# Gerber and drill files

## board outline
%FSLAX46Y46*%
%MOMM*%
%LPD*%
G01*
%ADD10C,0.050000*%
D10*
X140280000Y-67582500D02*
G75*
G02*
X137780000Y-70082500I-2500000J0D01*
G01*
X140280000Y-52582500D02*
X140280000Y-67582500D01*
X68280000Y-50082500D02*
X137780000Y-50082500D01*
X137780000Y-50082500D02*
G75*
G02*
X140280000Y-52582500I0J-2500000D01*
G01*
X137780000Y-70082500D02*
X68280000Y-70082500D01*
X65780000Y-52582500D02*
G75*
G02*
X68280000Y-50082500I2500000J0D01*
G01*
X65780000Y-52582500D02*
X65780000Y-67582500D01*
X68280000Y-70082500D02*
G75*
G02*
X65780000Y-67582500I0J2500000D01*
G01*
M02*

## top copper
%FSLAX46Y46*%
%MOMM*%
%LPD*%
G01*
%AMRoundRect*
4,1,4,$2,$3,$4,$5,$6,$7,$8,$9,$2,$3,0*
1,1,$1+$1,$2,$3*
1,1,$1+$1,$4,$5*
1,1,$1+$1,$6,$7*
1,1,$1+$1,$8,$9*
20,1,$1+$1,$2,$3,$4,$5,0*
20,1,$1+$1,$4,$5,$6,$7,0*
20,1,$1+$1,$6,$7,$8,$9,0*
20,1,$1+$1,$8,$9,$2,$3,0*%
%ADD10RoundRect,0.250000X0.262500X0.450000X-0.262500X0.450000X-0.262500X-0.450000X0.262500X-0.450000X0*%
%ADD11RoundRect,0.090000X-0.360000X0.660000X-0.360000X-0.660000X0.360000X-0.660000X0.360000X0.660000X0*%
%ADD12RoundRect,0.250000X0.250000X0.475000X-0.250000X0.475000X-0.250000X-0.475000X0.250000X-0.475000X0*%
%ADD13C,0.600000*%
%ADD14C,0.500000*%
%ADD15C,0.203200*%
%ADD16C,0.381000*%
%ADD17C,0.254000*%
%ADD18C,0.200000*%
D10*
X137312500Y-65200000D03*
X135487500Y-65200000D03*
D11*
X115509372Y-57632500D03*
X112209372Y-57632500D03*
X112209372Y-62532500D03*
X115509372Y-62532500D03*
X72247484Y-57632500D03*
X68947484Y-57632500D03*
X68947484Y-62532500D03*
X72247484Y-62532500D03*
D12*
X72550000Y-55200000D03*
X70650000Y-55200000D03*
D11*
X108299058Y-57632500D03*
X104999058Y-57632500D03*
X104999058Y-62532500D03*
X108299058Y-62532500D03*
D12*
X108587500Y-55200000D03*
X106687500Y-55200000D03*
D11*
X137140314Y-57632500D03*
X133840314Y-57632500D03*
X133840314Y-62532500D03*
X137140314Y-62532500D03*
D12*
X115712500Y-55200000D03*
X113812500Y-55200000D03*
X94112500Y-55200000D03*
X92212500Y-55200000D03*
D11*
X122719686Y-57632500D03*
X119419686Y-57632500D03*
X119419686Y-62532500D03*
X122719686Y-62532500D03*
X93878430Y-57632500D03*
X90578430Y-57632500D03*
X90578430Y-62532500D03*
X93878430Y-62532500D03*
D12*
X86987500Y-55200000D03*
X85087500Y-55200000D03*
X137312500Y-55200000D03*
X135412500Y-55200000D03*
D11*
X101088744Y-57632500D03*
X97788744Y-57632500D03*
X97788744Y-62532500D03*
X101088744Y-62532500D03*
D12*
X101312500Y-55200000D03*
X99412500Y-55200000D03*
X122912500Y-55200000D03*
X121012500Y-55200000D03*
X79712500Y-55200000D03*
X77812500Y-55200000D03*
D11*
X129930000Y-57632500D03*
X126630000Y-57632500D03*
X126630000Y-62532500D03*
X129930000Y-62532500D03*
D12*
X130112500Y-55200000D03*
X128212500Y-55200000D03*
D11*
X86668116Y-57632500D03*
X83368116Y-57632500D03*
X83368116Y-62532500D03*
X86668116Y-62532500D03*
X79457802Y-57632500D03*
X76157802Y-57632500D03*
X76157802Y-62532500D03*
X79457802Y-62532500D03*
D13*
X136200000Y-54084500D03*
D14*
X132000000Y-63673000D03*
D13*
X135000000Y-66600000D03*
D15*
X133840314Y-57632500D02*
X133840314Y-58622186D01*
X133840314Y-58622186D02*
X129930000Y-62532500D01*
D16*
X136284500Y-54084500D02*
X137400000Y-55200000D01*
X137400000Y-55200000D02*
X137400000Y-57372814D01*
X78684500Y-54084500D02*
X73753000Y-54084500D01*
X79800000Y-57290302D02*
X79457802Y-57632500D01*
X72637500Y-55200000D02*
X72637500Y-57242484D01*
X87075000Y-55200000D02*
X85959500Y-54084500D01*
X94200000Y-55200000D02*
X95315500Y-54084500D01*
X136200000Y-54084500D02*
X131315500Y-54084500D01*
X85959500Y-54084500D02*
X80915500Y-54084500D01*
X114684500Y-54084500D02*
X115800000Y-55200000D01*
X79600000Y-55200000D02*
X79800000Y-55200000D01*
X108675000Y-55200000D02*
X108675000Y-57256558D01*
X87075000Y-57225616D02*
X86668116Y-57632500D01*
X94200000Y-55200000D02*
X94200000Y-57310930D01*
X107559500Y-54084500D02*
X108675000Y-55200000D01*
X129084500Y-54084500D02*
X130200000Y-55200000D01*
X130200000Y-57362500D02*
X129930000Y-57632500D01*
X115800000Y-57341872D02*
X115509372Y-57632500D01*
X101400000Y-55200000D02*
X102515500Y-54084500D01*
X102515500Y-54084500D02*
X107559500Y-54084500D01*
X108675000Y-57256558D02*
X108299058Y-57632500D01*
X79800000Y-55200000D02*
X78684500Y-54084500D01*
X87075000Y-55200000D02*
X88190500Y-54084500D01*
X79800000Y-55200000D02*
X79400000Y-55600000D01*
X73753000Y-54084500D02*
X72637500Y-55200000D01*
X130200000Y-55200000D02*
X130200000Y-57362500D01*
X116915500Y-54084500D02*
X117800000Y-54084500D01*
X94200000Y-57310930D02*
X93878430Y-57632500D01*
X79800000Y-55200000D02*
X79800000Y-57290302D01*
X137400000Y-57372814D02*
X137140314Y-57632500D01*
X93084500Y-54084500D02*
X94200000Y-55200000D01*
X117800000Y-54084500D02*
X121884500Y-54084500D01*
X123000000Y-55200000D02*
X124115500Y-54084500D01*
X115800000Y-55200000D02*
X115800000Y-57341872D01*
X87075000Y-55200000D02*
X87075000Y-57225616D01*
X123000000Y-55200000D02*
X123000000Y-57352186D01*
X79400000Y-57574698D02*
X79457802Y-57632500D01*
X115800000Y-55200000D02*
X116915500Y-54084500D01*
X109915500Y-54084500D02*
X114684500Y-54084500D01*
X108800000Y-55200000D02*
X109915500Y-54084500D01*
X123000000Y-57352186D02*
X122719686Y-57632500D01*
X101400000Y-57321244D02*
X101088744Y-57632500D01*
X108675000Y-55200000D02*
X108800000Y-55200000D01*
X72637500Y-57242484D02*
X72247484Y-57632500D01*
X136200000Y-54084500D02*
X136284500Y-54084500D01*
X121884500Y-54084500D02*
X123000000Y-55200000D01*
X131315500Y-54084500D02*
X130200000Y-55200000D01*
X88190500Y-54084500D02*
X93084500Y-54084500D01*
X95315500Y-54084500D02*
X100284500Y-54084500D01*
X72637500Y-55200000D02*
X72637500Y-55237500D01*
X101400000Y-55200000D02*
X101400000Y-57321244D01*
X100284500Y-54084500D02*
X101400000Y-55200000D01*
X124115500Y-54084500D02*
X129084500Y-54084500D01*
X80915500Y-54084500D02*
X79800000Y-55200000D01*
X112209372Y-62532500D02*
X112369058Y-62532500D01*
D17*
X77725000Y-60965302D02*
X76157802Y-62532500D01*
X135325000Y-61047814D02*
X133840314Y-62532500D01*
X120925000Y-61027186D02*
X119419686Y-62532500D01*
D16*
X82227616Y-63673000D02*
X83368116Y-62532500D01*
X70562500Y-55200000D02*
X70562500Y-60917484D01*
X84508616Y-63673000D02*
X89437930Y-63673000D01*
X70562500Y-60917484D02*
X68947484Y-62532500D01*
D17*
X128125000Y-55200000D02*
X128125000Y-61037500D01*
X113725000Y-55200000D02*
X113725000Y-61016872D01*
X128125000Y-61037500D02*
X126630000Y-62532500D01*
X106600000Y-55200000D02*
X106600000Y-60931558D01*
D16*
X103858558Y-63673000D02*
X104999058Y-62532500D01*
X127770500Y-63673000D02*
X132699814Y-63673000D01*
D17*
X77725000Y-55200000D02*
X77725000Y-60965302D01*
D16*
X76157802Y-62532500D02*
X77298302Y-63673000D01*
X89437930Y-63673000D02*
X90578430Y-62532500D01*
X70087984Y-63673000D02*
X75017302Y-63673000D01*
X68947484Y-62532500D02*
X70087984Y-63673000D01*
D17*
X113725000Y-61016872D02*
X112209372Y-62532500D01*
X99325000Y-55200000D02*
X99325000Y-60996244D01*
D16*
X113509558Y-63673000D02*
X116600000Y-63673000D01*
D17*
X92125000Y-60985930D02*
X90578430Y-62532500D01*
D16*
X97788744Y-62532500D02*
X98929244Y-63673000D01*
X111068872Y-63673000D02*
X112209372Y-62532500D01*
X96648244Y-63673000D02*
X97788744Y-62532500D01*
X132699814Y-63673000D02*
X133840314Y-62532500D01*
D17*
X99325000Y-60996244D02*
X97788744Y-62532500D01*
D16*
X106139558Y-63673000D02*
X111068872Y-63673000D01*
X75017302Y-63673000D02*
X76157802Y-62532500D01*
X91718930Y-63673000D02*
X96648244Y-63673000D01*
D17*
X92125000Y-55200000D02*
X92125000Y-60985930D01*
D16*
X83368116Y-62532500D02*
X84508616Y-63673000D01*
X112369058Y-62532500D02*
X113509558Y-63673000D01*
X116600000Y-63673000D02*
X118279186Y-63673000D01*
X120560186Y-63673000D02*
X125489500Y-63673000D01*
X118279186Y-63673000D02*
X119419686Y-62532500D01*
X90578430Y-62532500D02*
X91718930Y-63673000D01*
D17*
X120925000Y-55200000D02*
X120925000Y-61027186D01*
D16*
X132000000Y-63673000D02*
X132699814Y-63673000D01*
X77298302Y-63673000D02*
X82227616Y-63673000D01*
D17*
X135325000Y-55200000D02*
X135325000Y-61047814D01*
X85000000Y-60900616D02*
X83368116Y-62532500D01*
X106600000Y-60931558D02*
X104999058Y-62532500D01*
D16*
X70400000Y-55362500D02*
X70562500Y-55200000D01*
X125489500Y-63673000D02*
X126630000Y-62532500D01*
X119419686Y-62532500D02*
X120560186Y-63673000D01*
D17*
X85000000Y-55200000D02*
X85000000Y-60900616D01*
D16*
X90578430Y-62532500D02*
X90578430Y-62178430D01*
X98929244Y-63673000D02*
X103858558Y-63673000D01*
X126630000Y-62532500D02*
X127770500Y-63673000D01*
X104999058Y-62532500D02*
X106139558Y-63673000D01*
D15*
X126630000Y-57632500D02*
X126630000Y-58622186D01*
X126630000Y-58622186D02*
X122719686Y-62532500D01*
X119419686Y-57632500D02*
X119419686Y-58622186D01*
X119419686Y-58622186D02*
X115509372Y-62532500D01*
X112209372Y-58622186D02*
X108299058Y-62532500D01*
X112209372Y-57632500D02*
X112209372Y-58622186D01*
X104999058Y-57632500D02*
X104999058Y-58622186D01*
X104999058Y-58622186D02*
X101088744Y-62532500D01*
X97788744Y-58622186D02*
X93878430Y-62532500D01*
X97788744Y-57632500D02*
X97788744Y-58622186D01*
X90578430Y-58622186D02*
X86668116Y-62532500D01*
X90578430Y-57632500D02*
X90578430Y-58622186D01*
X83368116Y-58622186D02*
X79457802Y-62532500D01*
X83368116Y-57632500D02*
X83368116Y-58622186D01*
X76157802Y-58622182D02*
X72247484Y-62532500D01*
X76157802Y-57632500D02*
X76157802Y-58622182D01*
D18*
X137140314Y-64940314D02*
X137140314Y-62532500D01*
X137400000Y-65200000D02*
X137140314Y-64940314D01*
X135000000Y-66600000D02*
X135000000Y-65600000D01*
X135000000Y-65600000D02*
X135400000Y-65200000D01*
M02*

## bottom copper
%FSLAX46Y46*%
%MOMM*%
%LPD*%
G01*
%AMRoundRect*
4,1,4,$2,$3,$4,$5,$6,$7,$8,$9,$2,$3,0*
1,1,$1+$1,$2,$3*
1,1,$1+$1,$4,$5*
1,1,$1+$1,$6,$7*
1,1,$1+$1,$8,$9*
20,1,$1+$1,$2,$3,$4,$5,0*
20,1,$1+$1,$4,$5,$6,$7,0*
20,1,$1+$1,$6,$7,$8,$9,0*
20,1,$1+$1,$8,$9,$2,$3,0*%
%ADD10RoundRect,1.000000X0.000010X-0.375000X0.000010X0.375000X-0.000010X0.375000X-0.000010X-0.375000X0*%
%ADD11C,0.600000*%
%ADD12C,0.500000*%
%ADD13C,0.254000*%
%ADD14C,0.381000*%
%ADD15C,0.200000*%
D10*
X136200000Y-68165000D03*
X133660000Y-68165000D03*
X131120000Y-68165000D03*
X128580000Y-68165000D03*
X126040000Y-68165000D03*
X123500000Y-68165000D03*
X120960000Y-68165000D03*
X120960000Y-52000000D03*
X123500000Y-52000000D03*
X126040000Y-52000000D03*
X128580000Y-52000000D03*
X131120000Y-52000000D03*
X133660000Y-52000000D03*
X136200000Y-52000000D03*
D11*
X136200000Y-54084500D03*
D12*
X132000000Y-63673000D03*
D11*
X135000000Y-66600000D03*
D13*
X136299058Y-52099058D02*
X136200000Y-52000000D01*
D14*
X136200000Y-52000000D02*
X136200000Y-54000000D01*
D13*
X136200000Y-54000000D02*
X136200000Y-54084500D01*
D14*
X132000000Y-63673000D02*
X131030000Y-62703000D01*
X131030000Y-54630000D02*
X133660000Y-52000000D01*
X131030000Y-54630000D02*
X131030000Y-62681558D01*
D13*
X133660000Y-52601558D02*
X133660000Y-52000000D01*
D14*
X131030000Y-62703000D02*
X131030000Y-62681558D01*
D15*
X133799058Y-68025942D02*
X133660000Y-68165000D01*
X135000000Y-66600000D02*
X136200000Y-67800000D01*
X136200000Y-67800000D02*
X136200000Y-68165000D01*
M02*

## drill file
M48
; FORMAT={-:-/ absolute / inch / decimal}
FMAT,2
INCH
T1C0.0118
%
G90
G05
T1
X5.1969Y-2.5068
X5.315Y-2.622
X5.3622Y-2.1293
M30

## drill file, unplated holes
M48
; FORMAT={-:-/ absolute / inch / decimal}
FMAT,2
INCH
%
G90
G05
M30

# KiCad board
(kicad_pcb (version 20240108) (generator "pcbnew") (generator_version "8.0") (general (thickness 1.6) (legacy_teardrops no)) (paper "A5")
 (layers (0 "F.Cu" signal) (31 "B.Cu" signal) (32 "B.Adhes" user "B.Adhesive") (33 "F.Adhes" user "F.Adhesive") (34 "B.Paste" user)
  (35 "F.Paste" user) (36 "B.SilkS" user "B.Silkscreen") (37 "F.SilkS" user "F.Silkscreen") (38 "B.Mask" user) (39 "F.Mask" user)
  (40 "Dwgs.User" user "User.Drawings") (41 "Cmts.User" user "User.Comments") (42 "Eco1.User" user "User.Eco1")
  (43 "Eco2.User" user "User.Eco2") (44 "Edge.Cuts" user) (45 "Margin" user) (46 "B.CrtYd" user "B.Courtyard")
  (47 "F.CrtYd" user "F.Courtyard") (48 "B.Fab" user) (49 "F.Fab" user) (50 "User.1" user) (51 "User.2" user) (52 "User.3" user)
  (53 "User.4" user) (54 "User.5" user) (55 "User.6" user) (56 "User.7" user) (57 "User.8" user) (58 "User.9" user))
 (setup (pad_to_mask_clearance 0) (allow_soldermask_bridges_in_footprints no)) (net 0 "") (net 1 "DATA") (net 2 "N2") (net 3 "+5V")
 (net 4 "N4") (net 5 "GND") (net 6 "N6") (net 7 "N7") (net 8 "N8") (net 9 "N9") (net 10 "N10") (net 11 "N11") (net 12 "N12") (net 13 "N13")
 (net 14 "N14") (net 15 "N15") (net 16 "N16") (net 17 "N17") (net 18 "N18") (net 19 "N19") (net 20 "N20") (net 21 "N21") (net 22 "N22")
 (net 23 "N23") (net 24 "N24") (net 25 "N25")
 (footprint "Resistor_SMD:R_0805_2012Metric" (layer "F.Cu") (at 136.4 65.2 180)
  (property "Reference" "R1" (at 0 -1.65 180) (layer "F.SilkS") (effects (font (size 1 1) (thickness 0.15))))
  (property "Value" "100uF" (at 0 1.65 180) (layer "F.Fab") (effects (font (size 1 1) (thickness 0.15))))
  (pad "1" smd roundrect (at -0.9125 0 180) (size 1.025 1.4) (layers "F.Cu" "F.Paste" "F.Mask") (roundrect_rratio 0.243902) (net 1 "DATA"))
  (pad "2" smd roundrect (at 0.9125 0 180) (size 1.025 1.4) (layers "F.Cu" "F.Paste" "F.Mask") (roundrect_rratio 0.243902) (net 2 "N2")))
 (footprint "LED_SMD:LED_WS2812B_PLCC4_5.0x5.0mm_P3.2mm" (layer "F.Cu") (at 113.859372 60.0825 -90)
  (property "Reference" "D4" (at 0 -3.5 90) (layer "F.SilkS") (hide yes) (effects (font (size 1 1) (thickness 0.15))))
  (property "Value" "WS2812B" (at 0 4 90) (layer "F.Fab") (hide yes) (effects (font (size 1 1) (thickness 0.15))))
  (pad "1" smd roundrect (at -2.45 -1.65 270) (size 1.5 0.9) (layers "F.Cu" "F.Paste" "F.Mask") (roundrect_rratio 0.1) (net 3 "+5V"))
  (pad "2" smd roundrect (at -2.45 1.65 270) (size 1.5 0.9) (layers "F.Cu" "F.Paste" "F.Mask") (roundrect_rratio 0.1) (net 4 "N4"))
  (pad "3" smd roundrect (at 2.45 1.65 270) (size 1.5 0.9) (layers "F.Cu" "F.Paste" "F.Mask") (roundrect_rratio 0.1) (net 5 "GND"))
  (pad "4" smd roundrect (at 2.45 -1.65 270) (size 1.5 0.9) (layers "F.Cu" "F.Paste" "F.Mask") (roundrect_rratio 0.1) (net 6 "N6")))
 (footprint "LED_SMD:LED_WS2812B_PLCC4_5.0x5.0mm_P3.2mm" (layer "F.Cu") (at 70.597484 60.0825 -90)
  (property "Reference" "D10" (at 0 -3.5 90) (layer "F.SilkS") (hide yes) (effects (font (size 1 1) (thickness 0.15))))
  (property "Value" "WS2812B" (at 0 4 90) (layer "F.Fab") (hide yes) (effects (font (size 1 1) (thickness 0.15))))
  (pad "1" smd roundrect (at -2.45 -1.65 270) (size 1.5 0.9) (layers "F.Cu" "F.Paste" "F.Mask") (roundrect_rratio 0.1) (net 3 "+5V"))
  (pad "2" smd roundrect (at -2.45 1.65 270) (size 1.5 0.9) (layers "F.Cu" "F.Paste" "F.Mask") (roundrect_rratio 0.1) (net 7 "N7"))
  (pad "3" smd roundrect (at 2.45 1.65 270) (size 1.5 0.9) (layers "F.Cu" "F.Paste" "F.Mask") (roundrect_rratio 0.1) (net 5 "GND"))
  (pad "4" smd roundrect (at 2.45 -1.65 270) (size 1.5 0.9) (layers "F.Cu" "F.Paste" "F.Mask") (roundrect_rratio 0.1) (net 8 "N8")))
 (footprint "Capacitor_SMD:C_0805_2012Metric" (layer "F.Cu") (at 71.6 55.2 180)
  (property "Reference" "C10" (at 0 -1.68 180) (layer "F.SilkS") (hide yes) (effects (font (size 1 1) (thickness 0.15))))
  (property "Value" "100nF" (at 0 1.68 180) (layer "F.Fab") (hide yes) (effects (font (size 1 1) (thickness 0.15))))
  (pad "1" smd roundrect (at -0.95 0 180) (size 1 1.45) (layers "F.Cu" "F.Paste" "F.Mask") (roundrect_rratio 0.25) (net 3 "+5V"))
  (pad "2" smd roundrect (at 0.95 0 180) (size 1 1.45) (layers "F.Cu" "F.Paste" "F.Mask") (roundrect_rratio 0.25) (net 5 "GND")))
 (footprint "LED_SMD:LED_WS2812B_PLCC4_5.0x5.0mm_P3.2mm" (layer "F.Cu") (at 106.649058 60.0825 -90)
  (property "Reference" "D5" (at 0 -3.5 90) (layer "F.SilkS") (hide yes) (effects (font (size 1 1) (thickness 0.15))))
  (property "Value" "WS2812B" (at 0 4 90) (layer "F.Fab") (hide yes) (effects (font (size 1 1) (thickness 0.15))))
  (pad "1" smd roundrect (at -2.45 -1.65 270) (size 1.5 0.9) (layers "F.Cu" "F.Paste" "F.Mask") (roundrect_rratio 0.1) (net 3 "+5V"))
  (pad "2" smd roundrect (at -2.45 1.65 270) (size 1.5 0.9) (layers "F.Cu" "F.Paste" "F.Mask") (roundrect_rratio 0.1) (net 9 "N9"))
  (pad "3" smd roundrect (at 2.45 1.65 270) (size 1.5 0.9) (layers "F.Cu" "F.Paste" "F.Mask") (roundrect_rratio 0.1) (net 5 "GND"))
  (pad "4" smd roundrect (at 2.45 -1.65 270) (size 1.5 0.9) (layers "F.Cu" "F.Paste" "F.Mask") (roundrect_rratio 0.1) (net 4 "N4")))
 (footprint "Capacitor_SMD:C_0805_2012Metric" (layer "F.Cu") (at 107.6375 55.2 180)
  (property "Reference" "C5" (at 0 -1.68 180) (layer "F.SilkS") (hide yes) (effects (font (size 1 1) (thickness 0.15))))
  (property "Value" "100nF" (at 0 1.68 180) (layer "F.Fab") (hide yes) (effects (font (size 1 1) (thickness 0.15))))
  (pad "1" smd roundrect (at -0.95 0 180) (size 1 1.45) (layers "F.Cu" "F.Paste" "F.Mask") (roundrect_rratio 0.25) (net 3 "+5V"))
  (pad "2" smd roundrect (at 0.95 0 180) (size 1 1.45) (layers "F.Cu" "F.Paste" "F.Mask") (roundrect_rratio 0.25) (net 5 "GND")))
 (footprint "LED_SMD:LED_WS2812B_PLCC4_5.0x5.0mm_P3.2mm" (layer "F.Cu") (at 135.490314 60.0825 -90)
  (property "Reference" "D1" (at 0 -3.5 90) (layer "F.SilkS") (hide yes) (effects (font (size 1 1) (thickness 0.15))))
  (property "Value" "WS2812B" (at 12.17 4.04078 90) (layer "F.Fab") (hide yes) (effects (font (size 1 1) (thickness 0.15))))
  (pad "1" smd roundrect (at -2.45 -1.65 270) (size 1.5 0.9) (layers "F.Cu" "F.Paste" "F.Mask") (roundrect_rratio 0.1) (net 3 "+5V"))
  (pad "2" smd roundrect (at -2.45 1.65 270) (size 1.5 0.9) (layers "F.Cu" "F.Paste" "F.Mask") (roundrect_rratio 0.1) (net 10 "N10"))
  (pad "3" smd roundrect (at 2.45 1.65 270) (size 1.5 0.9) (layers "F.Cu" "F.Paste" "F.Mask") (roundrect_rratio 0.1) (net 5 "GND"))
  (pad "4" smd roundrect (at 2.45 -1.65 270) (size 1.5 0.9) (layers "F.Cu" "F.Paste" "F.Mask") (roundrect_rratio 0.1) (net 1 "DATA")))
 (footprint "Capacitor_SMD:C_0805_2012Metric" (layer "F.Cu") (at 114.7625 55.2 180)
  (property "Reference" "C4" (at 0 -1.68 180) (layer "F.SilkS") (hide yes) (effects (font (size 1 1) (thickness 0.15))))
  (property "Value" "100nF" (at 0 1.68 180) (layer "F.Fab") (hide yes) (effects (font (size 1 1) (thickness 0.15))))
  (pad "1" smd roundrect (at -0.95 0 180) (size 1 1.45) (layers "F.Cu" "F.Paste" "F.Mask") (roundrect_rratio 0.25) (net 3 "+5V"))
  (pad "2" smd roundrect (at 0.95 0 180) (size 1 1.45) (layers "F.Cu" "F.Paste" "F.Mask") (roundrect_rratio 0.25) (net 5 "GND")))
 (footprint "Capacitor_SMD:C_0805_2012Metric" (layer "F.Cu") (at 93.1625 55.2 180)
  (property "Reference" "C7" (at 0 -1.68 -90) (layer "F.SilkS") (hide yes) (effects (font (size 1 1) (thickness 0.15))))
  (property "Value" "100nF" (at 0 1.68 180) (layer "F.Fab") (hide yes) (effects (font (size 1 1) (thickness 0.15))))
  (pad "1" smd roundrect (at -0.95 0 180) (size 1 1.45) (layers "F.Cu" "F.Paste" "F.Mask") (roundrect_rratio 0.25) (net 3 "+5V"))
  (pad "2" smd roundrect (at 0.95 0 180) (size 1 1.45) (layers "F.Cu" "F.Paste" "F.Mask") (roundrect_rratio 0.25) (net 5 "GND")))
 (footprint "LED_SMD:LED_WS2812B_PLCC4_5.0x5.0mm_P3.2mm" (layer "F.Cu") (at 121.069686 60.0825 -90)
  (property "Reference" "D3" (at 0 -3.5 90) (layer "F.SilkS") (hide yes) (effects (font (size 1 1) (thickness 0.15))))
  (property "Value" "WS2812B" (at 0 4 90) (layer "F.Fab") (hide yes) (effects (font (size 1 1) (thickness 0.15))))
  (pad "1" smd roundrect (at -2.45 -1.65 270) (size 1.5 0.9) (layers "F.Cu" "F.Paste" "F.Mask") (roundrect_rratio 0.1) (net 3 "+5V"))
  (pad "2" smd roundrect (at -2.45 1.65 270) (size 1.5 0.9) (layers "F.Cu" "F.Paste" "F.Mask") (roundrect_rratio 0.1) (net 6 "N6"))
  (pad "3" smd roundrect (at 2.45 1.65 270) (size 1.5 0.9) (layers "F.Cu" "F.Paste" "F.Mask") (roundrect_rratio 0.1) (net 5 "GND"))
  (pad "4" smd roundrect (at 2.45 -1.65 270) (size 1.5 0.9) (layers "F.Cu" "F.Paste" "F.Mask") (roundrect_rratio 0.1) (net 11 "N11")))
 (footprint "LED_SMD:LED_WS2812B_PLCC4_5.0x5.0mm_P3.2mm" (layer "F.Cu") (at 92.22843 60.0825 -90)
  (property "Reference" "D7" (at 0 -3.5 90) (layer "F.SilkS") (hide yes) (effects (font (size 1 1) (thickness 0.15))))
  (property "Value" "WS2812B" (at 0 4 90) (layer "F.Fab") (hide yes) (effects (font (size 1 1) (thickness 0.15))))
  (pad "1" smd roundrect (at -2.45 -1.65 270) (size 1.5 0.9) (layers "F.Cu" "F.Paste" "F.Mask") (roundrect_rratio 0.1) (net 3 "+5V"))
  (pad "2" smd roundrect (at -2.45 1.65 270) (size 1.5 0.9) (layers "F.Cu" "F.Paste" "F.Mask") (roundrect_rratio 0.1) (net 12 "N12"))
  (pad "3" smd roundrect (at 2.45 1.65 270) (size 1.5 0.9) (layers "F.Cu" "F.Paste" "F.Mask") (roundrect_rratio 0.1) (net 5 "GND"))
  (pad "4" smd roundrect (at 2.45 -1.65 270) (size 1.5 0.9) (layers "F.Cu" "F.Paste" "F.Mask") (roundrect_rratio 0.1) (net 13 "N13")))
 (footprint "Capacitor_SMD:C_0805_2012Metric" (layer "F.Cu") (at 86.0375 55.2 180)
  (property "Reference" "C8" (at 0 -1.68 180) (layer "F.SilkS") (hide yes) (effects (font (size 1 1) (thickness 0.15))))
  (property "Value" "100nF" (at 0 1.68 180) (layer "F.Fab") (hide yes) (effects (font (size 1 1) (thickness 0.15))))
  (pad "1" smd roundrect (at -0.95 0 180) (size 1 1.45) (layers "F.Cu" "F.Paste" "F.Mask") (roundrect_rratio 0.25) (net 3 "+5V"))
  (pad "2" smd roundrect (at 0.95 0 180) (size 1 1.45) (layers "F.Cu" "F.Paste" "F.Mask") (roundrect_rratio 0.25) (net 5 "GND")))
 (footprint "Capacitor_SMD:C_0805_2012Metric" (layer "F.Cu") (at 136.3625 55.2 180)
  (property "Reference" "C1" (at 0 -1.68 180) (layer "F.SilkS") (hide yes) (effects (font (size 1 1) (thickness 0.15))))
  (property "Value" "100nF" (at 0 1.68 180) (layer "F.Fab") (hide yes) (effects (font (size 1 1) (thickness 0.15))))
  (pad "1" smd roundrect (at -0.95 0 180) (size 1 1.45) (layers "F.Cu" "F.Paste" "F.Mask") (roundrect_rratio 0.25) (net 3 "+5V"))
  (pad "2" smd roundrect (at 0.95 0 180) (size 1 1.45) (layers "F.Cu" "F.Paste" "F.Mask") (roundrect_rratio 0.25) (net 5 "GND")))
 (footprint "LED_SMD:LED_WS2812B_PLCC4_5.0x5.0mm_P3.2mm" (layer "F.Cu") (at 99.438744 60.0825 -90)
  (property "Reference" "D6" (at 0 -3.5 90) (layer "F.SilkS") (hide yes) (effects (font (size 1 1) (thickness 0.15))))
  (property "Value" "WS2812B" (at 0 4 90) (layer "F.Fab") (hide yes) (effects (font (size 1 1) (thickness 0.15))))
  (pad "1" smd roundrect (at -2.45 -1.65 270) (size 1.5 0.9) (layers "F.Cu" "F.Paste" "F.Mask") (roundrect_rratio 0.1) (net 3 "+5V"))
  (pad "2" smd roundrect (at -2.45 1.65 270) (size 1.5 0.9) (layers "F.Cu" "F.Paste" "F.Mask") (roundrect_rratio 0.1) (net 13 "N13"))
  (pad "3" smd roundrect (at 2.45 1.65 270) (size 1.5 0.9) (layers "F.Cu" "F.Paste" "F.Mask") (roundrect_rratio 0.1) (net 5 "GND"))
  (pad "4" smd roundrect (at 2.45 -1.65 270) (size 1.5 0.9) (layers "F.Cu" "F.Paste" "F.Mask") (roundrect_rratio 0.1) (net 9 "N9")))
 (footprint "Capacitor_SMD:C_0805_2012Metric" (layer "F.Cu") (at 100.3625 55.2 180)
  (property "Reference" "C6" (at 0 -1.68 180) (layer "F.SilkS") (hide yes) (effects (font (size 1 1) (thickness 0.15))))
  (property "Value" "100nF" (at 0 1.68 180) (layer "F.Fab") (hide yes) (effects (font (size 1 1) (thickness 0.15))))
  (pad "1" smd roundrect (at -0.95 0 180) (size 1 1.45) (layers "F.Cu" "F.Paste" "F.Mask") (roundrect_rratio 0.25) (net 3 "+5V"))
  (pad "2" smd roundrect (at 0.95 0 180) (size 1 1.45) (layers "F.Cu" "F.Paste" "F.Mask") (roundrect_rratio 0.25) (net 5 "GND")))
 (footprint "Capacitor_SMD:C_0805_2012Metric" (layer "F.Cu") (at 121.9625 55.2 180)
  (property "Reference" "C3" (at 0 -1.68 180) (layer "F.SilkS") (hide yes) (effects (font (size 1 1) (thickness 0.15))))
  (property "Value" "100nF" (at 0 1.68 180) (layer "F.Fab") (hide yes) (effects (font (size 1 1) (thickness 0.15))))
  (pad "1" smd roundrect (at -0.95 0 180) (size 1 1.45) (layers "F.Cu" "F.Paste" "F.Mask") (roundrect_rratio 0.25) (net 3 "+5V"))
  (pad "2" smd roundrect (at 0.95 0 180) (size 1 1.45) (layers "F.Cu" "F.Paste" "F.Mask") (roundrect_rratio 0.25) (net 5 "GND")))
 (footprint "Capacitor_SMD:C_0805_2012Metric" (layer "F.Cu") (at 78.7625 55.2 180)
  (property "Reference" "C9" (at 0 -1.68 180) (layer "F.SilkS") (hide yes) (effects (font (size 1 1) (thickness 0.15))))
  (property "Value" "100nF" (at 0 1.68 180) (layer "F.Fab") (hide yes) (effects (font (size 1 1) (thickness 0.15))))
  (pad "1" smd roundrect (at -0.95 0 180) (size 1 1.45) (layers "F.Cu" "F.Paste" "F.Mask") (roundrect_rratio 0.25) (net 3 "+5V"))
  (pad "2" smd roundrect (at 0.95 0 180) (size 1 1.45) (layers "F.Cu" "F.Paste" "F.Mask") (roundrect_rratio 0.25) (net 5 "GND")))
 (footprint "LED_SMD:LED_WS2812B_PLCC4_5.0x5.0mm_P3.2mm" (layer "F.Cu") (at 128.28 60.0825 -90)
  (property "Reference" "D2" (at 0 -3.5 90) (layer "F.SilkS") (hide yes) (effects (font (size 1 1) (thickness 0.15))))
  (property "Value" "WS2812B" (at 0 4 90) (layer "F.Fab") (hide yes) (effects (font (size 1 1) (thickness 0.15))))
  (pad "1" smd roundrect (at -2.45 -1.65 270) (size 1.5 0.9) (layers "F.Cu" "F.Paste" "F.Mask") (roundrect_rratio 0.1) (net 3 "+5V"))
  (pad "2" smd roundrect (at -2.45 1.65 270) (size 1.5 0.9) (layers "F.Cu" "F.Paste" "F.Mask") (roundrect_rratio 0.1) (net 11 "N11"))
  (pad "3" smd roundrect (at 2.45 1.65 270) (size 1.5 0.9) (layers "F.Cu" "F.Paste" "F.Mask") (roundrect_rratio 0.1) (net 5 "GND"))
  (pad "4" smd roundrect (at 2.45 -1.65 270) (size 1.5 0.9) (layers "F.Cu" "F.Paste" "F.Mask") (roundrect_rratio 0.1) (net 10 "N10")))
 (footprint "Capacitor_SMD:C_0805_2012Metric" (layer "F.Cu") (at 129.1625 55.2 180)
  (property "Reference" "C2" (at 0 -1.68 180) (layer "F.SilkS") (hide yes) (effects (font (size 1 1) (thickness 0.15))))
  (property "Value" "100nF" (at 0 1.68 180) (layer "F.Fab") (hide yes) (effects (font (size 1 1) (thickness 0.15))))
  (pad "1" smd roundrect (at -0.95 0 180) (size 1 1.45) (layers "F.Cu" "F.Paste" "F.Mask") (roundrect_rratio 0.25) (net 3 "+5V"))
  (pad "2" smd roundrect (at 0.95 0 180) (size 1 1.45) (layers "F.Cu" "F.Paste" "F.Mask") (roundrect_rratio 0.25) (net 5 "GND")))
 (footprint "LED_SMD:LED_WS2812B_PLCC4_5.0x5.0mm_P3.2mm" (layer "F.Cu") (at 85.018116 60.0825 -90)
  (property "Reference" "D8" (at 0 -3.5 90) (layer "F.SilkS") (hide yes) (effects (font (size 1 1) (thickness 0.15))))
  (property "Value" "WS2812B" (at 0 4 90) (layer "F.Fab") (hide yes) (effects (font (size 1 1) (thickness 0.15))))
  (pad "1" smd roundrect (at -2.45 -1.65 270) (size 1.5 0.9) (layers "F.Cu" "F.Paste" "F.Mask") (roundrect_rratio 0.1) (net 3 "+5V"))
  (pad "2" smd roundrect (at -2.45 1.65 270) (size 1.5 0.9) (layers "F.Cu" "F.Paste" "F.Mask") (roundrect_rratio 0.1) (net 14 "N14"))
  (pad "3" smd roundrect (at 2.45 1.65 270) (size 1.5 0.9) (layers "F.Cu" "F.Paste" "F.Mask") (roundrect_rratio 0.1) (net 5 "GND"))
  (pad "4" smd roundrect (at 2.45 -1.65 270) (size 1.5 0.9) (layers "F.Cu" "F.Paste" "F.Mask") (roundrect_rratio 0.1) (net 12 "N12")))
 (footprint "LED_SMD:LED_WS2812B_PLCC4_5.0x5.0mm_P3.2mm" (layer "F.Cu") (at 77.807802 60.0825 -90)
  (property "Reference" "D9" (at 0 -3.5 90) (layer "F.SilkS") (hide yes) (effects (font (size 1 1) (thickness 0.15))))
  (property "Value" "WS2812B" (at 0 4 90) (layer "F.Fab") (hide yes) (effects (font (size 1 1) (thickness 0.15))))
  (pad "1" smd roundrect (at -2.45 -1.65 270) (size 1.5 0.9) (layers "F.Cu" "F.Paste" "F.Mask") (roundrect_rratio 0.1) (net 3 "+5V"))
  (pad "2" smd roundrect (at -2.45 1.65 270) (size 1.5 0.9) (layers "F.Cu" "F.Paste" "F.Mask") (roundrect_rratio 0.1) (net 8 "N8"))
  (pad "3" smd roundrect (at 2.45 1.65 270) (size 1.5 0.9) (layers "F.Cu" "F.Paste" "F.Mask") (roundrect_rratio 0.1) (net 5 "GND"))
  (pad "4" smd roundrect (at 2.45 -1.65 270) (size 1.5 0.9) (layers "F.Cu" "F.Paste" "F.Mask") (roundrect_rratio 0.1) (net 14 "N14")))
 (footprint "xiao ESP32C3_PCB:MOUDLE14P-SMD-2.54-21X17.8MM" (layer "B.Cu") (at 118.08 69 90)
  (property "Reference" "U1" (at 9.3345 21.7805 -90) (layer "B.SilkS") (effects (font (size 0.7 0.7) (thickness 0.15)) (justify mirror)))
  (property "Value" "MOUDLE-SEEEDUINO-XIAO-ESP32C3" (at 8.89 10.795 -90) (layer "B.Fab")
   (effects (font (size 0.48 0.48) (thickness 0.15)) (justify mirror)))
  (pad "1" smd roundrect (at 0.835 18.12 90) (size 2.75 2) (layers "B.Cu" "B.Paste" "B.Mask") (roundrect_rratio 0.5) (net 2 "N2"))
  (pad "2" smd roundrect (at 0.835 15.58 90) (size 2.75 2) (layers "B.Cu" "B.Paste" "B.Mask") (roundrect_rratio 0.5) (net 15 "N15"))
  (pad "3" smd roundrect (at 0.835 13.04 90) (size 2.75 2) (layers "B.Cu" "B.Paste" "B.Mask") (roundrect_rratio 0.5) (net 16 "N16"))
  (pad "4" smd roundrect (at 0.835 10.5 90) (size 2.75 2) (layers "B.Cu" "B.Paste" "B.Mask") (roundrect_rratio 0.5) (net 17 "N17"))
  (pad "5" smd roundrect (at 0.835 7.96 90) (size 2.75 2) (layers "B.Cu" "B.Paste" "B.Mask") (roundrect_rratio 0.5) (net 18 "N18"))
  (pad "6" smd roundrect (at 0.835 5.42 90) (size 2.75 2) (layers "B.Cu" "B.Paste" "B.Mask") (roundrect_rratio 0.5) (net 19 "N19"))
  (pad "7" smd roundrect (at 0.835 2.88 90) (size 2.75 2) (layers "B.Cu" "B.Paste" "B.Mask") (roundrect_rratio 0.5) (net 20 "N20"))
  (pad "8" smd roundrect (at 17 2.88 90) (size 2.75 2) (layers "B.Cu" "B.Paste" "B.Mask") (roundrect_rratio 0.5) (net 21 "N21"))
  (pad "9" smd roundrect (at 17 5.42 90) (size 2.75 2) (layers "B.Cu" "B.Paste" "B.Mask") (roundrect_rratio 0.5) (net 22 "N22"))
  (pad "10" smd roundrect (at 17 7.96 90) (size 2.75 2) (layers "B.Cu" "B.Paste" "B.Mask") (roundrect_rratio 0.5) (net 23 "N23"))
  (pad "11" smd roundrect (at 17 10.5 90) (size 2.75 2) (layers "B.Cu" "B.Paste" "B.Mask") (roundrect_rratio 0.5) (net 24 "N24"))
  (pad "12" smd roundrect (at 17 13.04 90) (size 2.75 2) (layers "B.Cu" "B.Paste" "B.Mask") (roundrect_rratio 0.5) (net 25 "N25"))
  (pad "13" smd roundrect (at 17 15.58 90) (size 2.75 2) (layers "B.Cu" "B.Paste" "B.Mask") (roundrect_rratio 0.5) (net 5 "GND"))
  (pad "14" smd roundrect (at 17 18.12 90) (size 2.75 2) (layers "B.Cu" "B.Paste" "B.Mask") (roundrect_rratio 0.5) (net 3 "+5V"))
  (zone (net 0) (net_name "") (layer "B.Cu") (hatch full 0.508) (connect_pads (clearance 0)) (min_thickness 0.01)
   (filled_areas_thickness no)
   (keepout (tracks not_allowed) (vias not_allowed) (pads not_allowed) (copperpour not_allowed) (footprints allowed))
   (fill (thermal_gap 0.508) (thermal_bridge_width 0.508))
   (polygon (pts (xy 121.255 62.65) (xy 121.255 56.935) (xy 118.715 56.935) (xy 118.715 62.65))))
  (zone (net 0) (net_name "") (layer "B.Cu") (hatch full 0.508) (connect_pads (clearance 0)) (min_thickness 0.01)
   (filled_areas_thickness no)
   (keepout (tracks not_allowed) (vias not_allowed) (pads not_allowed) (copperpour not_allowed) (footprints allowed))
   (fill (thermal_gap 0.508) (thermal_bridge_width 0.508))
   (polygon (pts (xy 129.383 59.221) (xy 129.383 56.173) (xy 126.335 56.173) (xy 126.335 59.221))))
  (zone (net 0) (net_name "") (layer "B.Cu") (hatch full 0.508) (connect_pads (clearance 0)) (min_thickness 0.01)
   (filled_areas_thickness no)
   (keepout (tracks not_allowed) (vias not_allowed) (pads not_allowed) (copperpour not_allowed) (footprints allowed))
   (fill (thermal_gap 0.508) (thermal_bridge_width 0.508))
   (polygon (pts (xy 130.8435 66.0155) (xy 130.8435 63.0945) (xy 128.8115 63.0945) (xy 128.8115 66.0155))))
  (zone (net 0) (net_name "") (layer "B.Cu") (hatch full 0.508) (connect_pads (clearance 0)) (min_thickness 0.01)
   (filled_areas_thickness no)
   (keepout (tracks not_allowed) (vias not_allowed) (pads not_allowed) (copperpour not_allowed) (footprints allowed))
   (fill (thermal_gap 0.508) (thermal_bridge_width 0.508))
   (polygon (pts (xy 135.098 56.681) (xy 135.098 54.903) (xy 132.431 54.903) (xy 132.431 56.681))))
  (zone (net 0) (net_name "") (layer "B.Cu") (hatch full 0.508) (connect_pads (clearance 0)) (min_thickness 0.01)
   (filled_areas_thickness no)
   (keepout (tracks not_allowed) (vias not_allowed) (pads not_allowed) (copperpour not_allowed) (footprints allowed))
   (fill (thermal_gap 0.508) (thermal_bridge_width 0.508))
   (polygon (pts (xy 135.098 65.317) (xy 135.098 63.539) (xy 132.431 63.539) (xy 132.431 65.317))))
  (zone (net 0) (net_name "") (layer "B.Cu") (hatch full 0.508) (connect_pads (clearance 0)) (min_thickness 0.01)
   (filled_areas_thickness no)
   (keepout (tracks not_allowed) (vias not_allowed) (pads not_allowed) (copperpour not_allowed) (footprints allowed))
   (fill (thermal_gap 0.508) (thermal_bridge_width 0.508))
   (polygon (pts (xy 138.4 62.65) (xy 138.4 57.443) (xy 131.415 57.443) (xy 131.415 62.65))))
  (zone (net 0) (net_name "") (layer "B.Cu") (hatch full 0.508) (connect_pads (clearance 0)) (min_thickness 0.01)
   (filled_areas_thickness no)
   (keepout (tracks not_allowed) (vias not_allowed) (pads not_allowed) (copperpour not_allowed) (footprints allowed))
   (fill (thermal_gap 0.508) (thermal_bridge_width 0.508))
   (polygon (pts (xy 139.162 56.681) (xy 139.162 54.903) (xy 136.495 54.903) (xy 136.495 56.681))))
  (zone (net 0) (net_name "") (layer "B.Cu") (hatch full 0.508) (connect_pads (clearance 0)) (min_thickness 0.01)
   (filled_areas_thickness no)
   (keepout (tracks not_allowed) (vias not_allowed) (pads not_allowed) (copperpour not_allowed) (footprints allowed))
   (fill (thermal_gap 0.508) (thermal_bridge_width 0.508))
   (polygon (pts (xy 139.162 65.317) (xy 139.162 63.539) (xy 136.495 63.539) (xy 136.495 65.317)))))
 (gr_arc (start 140.28 67.5825) (mid 139.547767 69.350267) (end 137.78 70.0825) (stroke (width 0.05) (type default)) (layer "Edge.Cuts"))
 (gr_line (start 140.28 52.5825) (end 140.28 67.5825) (stroke (width 0.05) (type default)) (layer "Edge.Cuts"))
 (gr_line (start 68.28 50.0825) (end 137.78 50.0825) (stroke (width 0.05) (type default)) (layer "Edge.Cuts"))
 (gr_arc (start 137.78 50.0825) (mid 139.547767 50.814733) (end 140.28 52.5825) (stroke (width 0.05) (type default)) (layer "Edge.Cuts"))
 (gr_line (start 137.78 70.0825) (end 68.28 70.0825) (stroke (width 0.05) (type default)) (layer "Edge.Cuts"))
 (gr_arc (start 65.78 52.5825) (mid 66.512233 50.814733) (end 68.28 50.0825) (stroke (width 0.05) (type default)) (layer "Edge.Cuts"))
 (gr_line (start 65.78 52.5825) (end 65.78 67.5825) (stroke (width 0.05) (type default)) (layer "Edge.Cuts"))
 (gr_arc (start 68.28 70.0825) (mid 66.512233 69.350267) (end 65.78 67.5825) (stroke (width 0.05) (type default)) (layer "Edge.Cuts"))
 (segment (start 133.840314 57.6325) (end 133.840314 58.622186) (width 0.2032) (layer "F.Cu") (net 10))
 (segment (start 133.840314 58.622186) (end 129.93 62.5325) (width 0.2032) (layer "F.Cu") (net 10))
 (segment (start 136.2845 54.0845) (end 137.4 55.2) (width 0.381) (layer "F.Cu") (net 3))
 (segment (start 137.4 55.2) (end 137.4 57.372814) (width 0.381) (layer "F.Cu") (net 3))
 (segment (start 78.6845 54.0845) (end 73.753 54.0845) (width 0.381) (layer "F.Cu") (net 3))
 (segment (start 79.8 57.290302) (end 79.457802 57.6325) (width 0.381) (layer "F.Cu") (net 3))
 (segment (start 72.6375 55.2) (end 72.6375 57.242484) (width 0.381) (layer "F.Cu") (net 3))
 (segment (start 87.075 55.2) (end 85.9595 54.0845) (width 0.381) (layer "F.Cu") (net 3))
 (segment (start 94.2 55.2) (end 95.3155 54.0845) (width 0.381) (layer "F.Cu") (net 3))
 (segment (start 136.2 54.0845) (end 131.3155 54.0845) (width 0.381) (layer "F.Cu") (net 3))
 (segment (start 85.9595 54.0845) (end 80.9155 54.0845) (width 0.381) (layer "F.Cu") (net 3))
 (segment (start 114.6845 54.0845) (end 115.8 55.2) (width 0.381) (layer "F.Cu") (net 3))
 (segment (start 79.6 55.2) (end 79.8 55.2) (width 0.381) (layer "F.Cu") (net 3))
 (segment (start 108.675 55.2) (end 108.675 57.256558) (width 0.381) (layer "F.Cu") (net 3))
 (segment (start 87.075 57.225616) (end 86.668116 57.6325) (width 0.381) (layer "F.Cu") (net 3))
 (segment (start 94.2 55.2) (end 94.2 57.31093) (width 0.381) (layer "F.Cu") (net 3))
 (segment (start 107.5595 54.0845) (end 108.675 55.2) (width 0.381) (layer "F.Cu") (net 3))
 (segment (start 129.0845 54.0845) (end 130.2 55.2) (width 0.381) (layer "F.Cu") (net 3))
 (segment (start 130.2 57.3625) (end 129.93 57.6325) (width 0.381) (layer "F.Cu") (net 3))
 (segment (start 115.8 57.341872) (end 115.509372 57.6325) (width 0.381) (layer "F.Cu") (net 3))
 (segment (start 101.4 55.2) (end 102.5155 54.0845) (width 0.381) (layer "F.Cu") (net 3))
 (segment (start 102.5155 54.0845) (end 107.5595 54.0845) (width 0.381) (layer "F.Cu") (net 3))
 (segment (start 108.675 57.256558) (end 108.299058 57.6325) (width 0.381) (layer "F.Cu") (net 3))
 (segment (start 79.8 55.2) (end 78.6845 54.0845) (width 0.381) (layer "F.Cu") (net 3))
 (segment (start 87.075 55.2) (end 88.1905 54.0845) (width 0.381) (layer "F.Cu") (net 3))
 (segment (start 79.8 55.2) (end 79.4 55.6) (width 0.381) (layer "F.Cu") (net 3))
 (segment (start 73.753 54.0845) (end 72.6375 55.2) (width 0.381) (layer "F.Cu") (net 3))
 (segment (start 130.2 55.2) (end 130.2 57.3625) (width 0.381) (layer "F.Cu") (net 3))
 (segment (start 116.9155 54.0845) (end 117.8 54.0845) (width 0.381) (layer "F.Cu") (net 3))
 (segment (start 94.2 57.31093) (end 93.87843 57.6325) (width 0.381) (layer "F.Cu") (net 3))
 (segment (start 79.8 55.2) (end 79.8 57.290302) (width 0.381) (layer "F.Cu") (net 3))
 (segment (start 137.4 57.372814) (end 137.140314 57.6325) (width 0.381) (layer "F.Cu") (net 3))
 (segment (start 93.0845 54.0845) (end 94.2 55.2) (width 0.381) (layer "F.Cu") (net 3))
 (segment (start 117.8 54.0845) (end 121.8845 54.0845) (width 0.381) (layer "F.Cu") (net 3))
 (segment (start 123 55.2) (end 124.1155 54.0845) (width 0.381) (layer "F.Cu") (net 3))
 (segment (start 115.8 55.2) (end 115.8 57.341872) (width 0.381) (layer "F.Cu") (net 3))
 (segment (start 87.075 55.2) (end 87.075 57.225616) (width 0.381) (layer "F.Cu") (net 3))
 (segment (start 123 55.2) (end 123 57.352186) (width 0.381) (layer "F.Cu") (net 3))
 (segment (start 79.4 57.574698) (end 79.457802 57.6325) (width 0.381) (layer "F.Cu") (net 3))
 (segment (start 115.8 55.2) (end 116.9155 54.0845) (width 0.381) (layer "F.Cu") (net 3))
 (segment (start 109.9155 54.0845) (end 114.6845 54.0845) (width 0.381) (layer "F.Cu") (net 3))
 (segment (start 108.8 55.2) (end 109.9155 54.0845) (width 0.381) (layer "F.Cu") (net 3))
 (segment (start 123 57.352186) (end 122.719686 57.6325) (width 0.381) (layer "F.Cu") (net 3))
 (segment (start 101.4 57.321244) (end 101.088744 57.6325) (width 0.381) (layer "F.Cu") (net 3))
 (segment (start 108.675 55.2) (end 108.8 55.2) (width 0.381) (layer "F.Cu") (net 3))
 (segment (start 72.6375 57.242484) (end 72.247484 57.6325) (width 0.381) (layer "F.Cu") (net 3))
 (segment (start 136.2 54.0845) (end 136.2845 54.0845) (width 0.381) (layer "F.Cu") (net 3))
 (segment (start 121.8845 54.0845) (end 123 55.2) (width 0.381) (layer "F.Cu") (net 3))
 (segment (start 131.3155 54.0845) (end 130.2 55.2) (width 0.381) (layer "F.Cu") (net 3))
 (segment (start 88.1905 54.0845) (end 93.0845 54.0845) (width 0.381) (layer "F.Cu") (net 3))
 (segment (start 95.3155 54.0845) (end 100.2845 54.0845) (width 0.381) (layer "F.Cu") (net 3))
 (segment (start 72.6375 55.2) (end 72.6375 55.2375) (width 0.381) (layer "F.Cu") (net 3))
 (segment (start 101.4 55.2) (end 101.4 57.321244) (width 0.381) (layer "F.Cu") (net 3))
 (segment (start 100.2845 54.0845) (end 101.4 55.2) (width 0.381) (layer "F.Cu") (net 3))
 (segment (start 124.1155 54.0845) (end 129.0845 54.0845) (width 0.381) (layer "F.Cu") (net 3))
 (segment (start 80.9155 54.0845) (end 79.8 55.2) (width 0.381) (layer "F.Cu") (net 3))
 (via (at 136.2 54.0845) (size 0.6) (drill 0.3) (layers "F.Cu" "B.Cu") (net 3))
 (segment (start 136.299058 52.099058) (end 136.2 52) (width 0.254) (layer "B.Cu") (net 3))
 (segment (start 136.2 52) (end 136.2 54) (width 0.381) (layer "B.Cu") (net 3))
 (segment (start 136.2 54) (end 136.2 54.0845) (width 0.254) (layer "B.Cu") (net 3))
 (segment (start 112.209372 62.5325) (end 112.369058 62.5325) (width 0.381) (layer "F.Cu") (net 5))
 (segment (start 77.725 60.965302) (end 76.157802 62.5325) (width 0.254) (layer "F.Cu") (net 5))
 (segment (start 135.325 61.047814) (end 133.840314 62.5325) (width 0.254) (layer "F.Cu") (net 5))
 (segment (start 120.925 61.027186) (end 119.419686 62.5325) (width 0.254) (layer "F.Cu") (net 5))
 (segment (start 82.227616 63.673) (end 83.368116 62.5325) (width 0.381) (layer "F.Cu") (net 5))
 (segment (start 70.5625 55.2) (end 70.5625 60.917484) (width 0.381) (layer "F.Cu") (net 5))
 (segment (start 84.508616 63.673) (end 89.43793 63.673) (width 0.381) (layer "F.Cu") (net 5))
 (segment (start 70.5625 60.917484) (end 68.947484 62.5325) (width 0.381) (layer "F.Cu") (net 5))
 (segment (start 128.125 55.2) (end 128.125 61.0375) (width 0.254) (layer "F.Cu") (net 5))
 (segment (start 113.725 55.2) (end 113.725 61.016872) (width 0.254) (layer "F.Cu") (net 5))
 (segment (start 128.125 61.0375) (end 126.63 62.5325) (width 0.254) (layer "F.Cu") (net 5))
 (segment (start 106.6 55.2) (end 106.6 60.931558) (width 0.254) (layer "F.Cu") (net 5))
 (segment (start 103.858558 63.673) (end 104.999058 62.5325) (width 0.381) (layer "F.Cu") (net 5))
 (segment (start 127.7705 63.673) (end 132.699814 63.673) (width 0.381) (layer "F.Cu") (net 5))
 (segment (start 77.725 55.2) (end 77.725 60.965302) (width 0.254) (layer "F.Cu") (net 5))
 (segment (start 76.157802 62.5325) (end 77.298302 63.673) (width 0.381) (layer "F.Cu") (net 5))
 (segment (start 89.43793 63.673) (end 90.57843 62.5325) (width 0.381) (layer "F.Cu") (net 5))
 (segment (start 70.087984 63.673) (end 75.017302 63.673) (width 0.381) (layer "F.Cu") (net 5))
 (segment (start 68.947484 62.5325) (end 70.087984 63.673) (width 0.381) (layer "F.Cu") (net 5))
 (segment (start 113.725 61.016872) (end 112.209372 62.5325) (width 0.254) (layer "F.Cu") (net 5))
 (segment (start 99.325 55.2) (end 99.325 60.996244) (width 0.254) (layer "F.Cu") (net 5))
 (segment (start 113.509558 63.673) (end 116.6 63.673) (width 0.381) (layer "F.Cu") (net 5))
 (segment (start 92.125 60.98593) (end 90.57843 62.5325) (width 0.254) (layer "F.Cu") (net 5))
 (segment (start 97.788744 62.5325) (end 98.929244 63.673) (width 0.381) (layer "F.Cu") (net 5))
 (segment (start 111.068872 63.673) (end 112.209372 62.5325) (width 0.381) (layer "F.Cu") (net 5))
 (segment (start 96.648244 63.673) (end 97.788744 62.5325) (width 0.381) (layer "F.Cu") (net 5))
 (segment (start 132.699814 63.673) (end 133.840314 62.5325) (width 0.381) (layer "F.Cu") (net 5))
 (segment (start 99.325 60.996244) (end 97.788744 62.5325) (width 0.254) (layer "F.Cu") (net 5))
 (segment (start 106.139558 63.673) (end 111.068872 63.673) (width 0.381) (layer "F.Cu") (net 5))
 (segment (start 75.017302 63.673) (end 76.157802 62.5325) (width 0.381) (layer "F.Cu") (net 5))
 (segment (start 91.71893 63.673) (end 96.648244 63.673) (width 0.381) (layer "F.Cu") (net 5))
 (segment (start 92.125 55.2) (end 92.125 60.98593) (width 0.254) (layer "F.Cu") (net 5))
 (segment (start 83.368116 62.5325) (end 84.508616 63.673) (width 0.381) (layer "F.Cu") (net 5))
 (segment (start 112.369058 62.5325) (end 113.509558 63.673) (width 0.381) (layer "F.Cu") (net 5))
 (segment (start 116.6 63.673) (end 118.279186 63.673) (width 0.381) (layer "F.Cu") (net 5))
 (segment (start 120.560186 63.673) (end 125.4895 63.673) (width 0.381) (layer "F.Cu") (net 5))
 (segment (start 118.279186 63.673) (end 119.419686 62.5325) (width 0.381) (layer "F.Cu") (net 5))
 (segment (start 90.57843 62.5325) (end 91.71893 63.673) (width 0.381) (layer "F.Cu") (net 5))
 (segment (start 120.925 55.2) (end 120.925 61.027186) (width 0.254) (layer "F.Cu") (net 5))
 (segment (start 132 63.673) (end 132.699814 63.673) (width 0.381) (layer "F.Cu") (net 5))
 (segment (start 77.298302 63.673) (end 82.227616 63.673) (width 0.381) (layer "F.Cu") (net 5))
 (segment (start 135.325 55.2) (end 135.325 61.047814) (width 0.254) (layer "F.Cu") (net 5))
 (segment (start 85 60.900616) (end 83.368116 62.5325) (width 0.254) (layer "F.Cu") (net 5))
 (segment (start 106.6 60.931558) (end 104.999058 62.5325) (width 0.254) (layer "F.Cu") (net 5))
 (segment (start 70.4 55.3625) (end 70.5625 55.2) (width 0.381) (layer "F.Cu") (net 5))
 (segment (start 125.4895 63.673) (end 126.63 62.5325) (width 0.381) (layer "F.Cu") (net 5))
 (segment (start 119.419686 62.5325) (end 120.560186 63.673) (width 0.381) (layer "F.Cu") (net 5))
 (segment (start 85 55.2) (end 85 60.900616) (width 0.254) (layer "F.Cu") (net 5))
 (segment (start 90.57843 62.5325) (end 90.57843 62.17843) (width 0.381) (layer "F.Cu") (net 5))
 (segment (start 98.929244 63.673) (end 103.858558 63.673) (width 0.381) (layer "F.Cu") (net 5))
 (segment (start 126.63 62.5325) (end 127.7705 63.673) (width 0.381) (layer "F.Cu") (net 5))
 (segment (start 104.999058 62.5325) (end 106.139558 63.673) (width 0.381) (layer "F.Cu") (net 5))
 (via (at 132 63.673) (size 0.5) (drill 0.3) (layers "F.Cu" "B.Cu") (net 5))
 (segment (start 132 63.673) (end 131.03 62.703) (width 0.381) (layer "B.Cu") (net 5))
 (segment (start 131.03 54.63) (end 133.66 52) (width 0.381) (layer "B.Cu") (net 5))
 (segment (start 131.03 54.63) (end 131.03 62.681558) (width 0.381) (layer "B.Cu") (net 5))
 (segment (start 133.66 52.601558) (end 133.66 52) (width 0.254) (layer "B.Cu") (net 5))
 (segment (start 131.03 62.703) (end 131.03 62.681558) (width 0.381) (layer "B.Cu") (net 5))
 (segment (start 126.63 57.6325) (end 126.63 58.622186) (width 0.2032) (layer "F.Cu") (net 11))
 (segment (start 126.63 58.622186) (end 122.719686 62.5325) (width 0.2032) (layer "F.Cu") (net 11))
 (segment (start 119.419686 57.6325) (end 119.419686 58.622186) (width 0.2032) (layer "F.Cu") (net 6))
 (segment (start 119.419686 58.622186) (end 115.509372 62.5325) (width 0.2032) (layer "F.Cu") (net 6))
 (segment (start 112.209372 58.622186) (end 108.299058 62.5325) (width 0.2032) (layer "F.Cu") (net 4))
 (segment (start 112.209372 57.6325) (end 112.209372 58.622186) (width 0.2032) (layer "F.Cu") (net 4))
 (segment (start 104.999058 57.6325) (end 104.999058 58.622186) (width 0.2032) (layer "F.Cu") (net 9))
 (segment (start 104.999058 58.622186) (end 101.088744 62.5325) (width 0.2032) (layer "F.Cu") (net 9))
 (segment (start 97.788744 58.622186) (end 93.87843 62.5325) (width 0.2032) (layer "F.Cu") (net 13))
 (segment (start 97.788744 57.6325) (end 97.788744 58.622186) (width 0.2032) (layer "F.Cu") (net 13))
 (segment (start 90.57843 58.622186) (end 86.668116 62.5325) (width 0.2032) (layer "F.Cu") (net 12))
 (segment (start 90.57843 57.6325) (end 90.57843 58.622186) (width 0.2032) (layer "F.Cu") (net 12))
 (segment (start 83.368116 58.622186) (end 79.457802 62.5325) (width 0.2032) (layer "F.Cu") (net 14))
 (segment (start 83.368116 57.6325) (end 83.368116 58.622186) (width 0.2032) (layer "F.Cu") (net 14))
 (segment (start 76.157802 58.622182) (end 72.247484 62.5325) (width 0.2032) (layer "F.Cu") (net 8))
 (segment (start 76.157802 57.6325) (end 76.157802 58.622182) (width 0.2032) (layer "F.Cu") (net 8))
 (segment (start 137.140314 64.940314) (end 137.140314 62.5325) (width 0.2) (layer "F.Cu") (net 1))
 (segment (start 137.4 65.2) (end 137.140314 64.940314) (width 0.2) (layer "F.Cu") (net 1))
 (segment (start 133.799058 68.025942) (end 133.66 68.165) (width 0.2) (layer "B.Cu") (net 15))
 (segment (start 135 66.6) (end 135 65.6) (width 0.2) (layer "F.Cu") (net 2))
 (segment (start 135 65.6) (end 135.4 65.2) (width 0.2) (layer "F.Cu") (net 2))
 (via (at 135 66.6) (size 0.6) (drill 0.3) (layers "F.Cu" "B.Cu") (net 2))
 (segment (start 135 66.6) (end 136.2 67.8) (width 0.2) (layer "B.Cu") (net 2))
 (segment (start 136.2 67.8) (end 136.2 68.165) (width 0.2) (layer "B.Cu") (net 2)))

